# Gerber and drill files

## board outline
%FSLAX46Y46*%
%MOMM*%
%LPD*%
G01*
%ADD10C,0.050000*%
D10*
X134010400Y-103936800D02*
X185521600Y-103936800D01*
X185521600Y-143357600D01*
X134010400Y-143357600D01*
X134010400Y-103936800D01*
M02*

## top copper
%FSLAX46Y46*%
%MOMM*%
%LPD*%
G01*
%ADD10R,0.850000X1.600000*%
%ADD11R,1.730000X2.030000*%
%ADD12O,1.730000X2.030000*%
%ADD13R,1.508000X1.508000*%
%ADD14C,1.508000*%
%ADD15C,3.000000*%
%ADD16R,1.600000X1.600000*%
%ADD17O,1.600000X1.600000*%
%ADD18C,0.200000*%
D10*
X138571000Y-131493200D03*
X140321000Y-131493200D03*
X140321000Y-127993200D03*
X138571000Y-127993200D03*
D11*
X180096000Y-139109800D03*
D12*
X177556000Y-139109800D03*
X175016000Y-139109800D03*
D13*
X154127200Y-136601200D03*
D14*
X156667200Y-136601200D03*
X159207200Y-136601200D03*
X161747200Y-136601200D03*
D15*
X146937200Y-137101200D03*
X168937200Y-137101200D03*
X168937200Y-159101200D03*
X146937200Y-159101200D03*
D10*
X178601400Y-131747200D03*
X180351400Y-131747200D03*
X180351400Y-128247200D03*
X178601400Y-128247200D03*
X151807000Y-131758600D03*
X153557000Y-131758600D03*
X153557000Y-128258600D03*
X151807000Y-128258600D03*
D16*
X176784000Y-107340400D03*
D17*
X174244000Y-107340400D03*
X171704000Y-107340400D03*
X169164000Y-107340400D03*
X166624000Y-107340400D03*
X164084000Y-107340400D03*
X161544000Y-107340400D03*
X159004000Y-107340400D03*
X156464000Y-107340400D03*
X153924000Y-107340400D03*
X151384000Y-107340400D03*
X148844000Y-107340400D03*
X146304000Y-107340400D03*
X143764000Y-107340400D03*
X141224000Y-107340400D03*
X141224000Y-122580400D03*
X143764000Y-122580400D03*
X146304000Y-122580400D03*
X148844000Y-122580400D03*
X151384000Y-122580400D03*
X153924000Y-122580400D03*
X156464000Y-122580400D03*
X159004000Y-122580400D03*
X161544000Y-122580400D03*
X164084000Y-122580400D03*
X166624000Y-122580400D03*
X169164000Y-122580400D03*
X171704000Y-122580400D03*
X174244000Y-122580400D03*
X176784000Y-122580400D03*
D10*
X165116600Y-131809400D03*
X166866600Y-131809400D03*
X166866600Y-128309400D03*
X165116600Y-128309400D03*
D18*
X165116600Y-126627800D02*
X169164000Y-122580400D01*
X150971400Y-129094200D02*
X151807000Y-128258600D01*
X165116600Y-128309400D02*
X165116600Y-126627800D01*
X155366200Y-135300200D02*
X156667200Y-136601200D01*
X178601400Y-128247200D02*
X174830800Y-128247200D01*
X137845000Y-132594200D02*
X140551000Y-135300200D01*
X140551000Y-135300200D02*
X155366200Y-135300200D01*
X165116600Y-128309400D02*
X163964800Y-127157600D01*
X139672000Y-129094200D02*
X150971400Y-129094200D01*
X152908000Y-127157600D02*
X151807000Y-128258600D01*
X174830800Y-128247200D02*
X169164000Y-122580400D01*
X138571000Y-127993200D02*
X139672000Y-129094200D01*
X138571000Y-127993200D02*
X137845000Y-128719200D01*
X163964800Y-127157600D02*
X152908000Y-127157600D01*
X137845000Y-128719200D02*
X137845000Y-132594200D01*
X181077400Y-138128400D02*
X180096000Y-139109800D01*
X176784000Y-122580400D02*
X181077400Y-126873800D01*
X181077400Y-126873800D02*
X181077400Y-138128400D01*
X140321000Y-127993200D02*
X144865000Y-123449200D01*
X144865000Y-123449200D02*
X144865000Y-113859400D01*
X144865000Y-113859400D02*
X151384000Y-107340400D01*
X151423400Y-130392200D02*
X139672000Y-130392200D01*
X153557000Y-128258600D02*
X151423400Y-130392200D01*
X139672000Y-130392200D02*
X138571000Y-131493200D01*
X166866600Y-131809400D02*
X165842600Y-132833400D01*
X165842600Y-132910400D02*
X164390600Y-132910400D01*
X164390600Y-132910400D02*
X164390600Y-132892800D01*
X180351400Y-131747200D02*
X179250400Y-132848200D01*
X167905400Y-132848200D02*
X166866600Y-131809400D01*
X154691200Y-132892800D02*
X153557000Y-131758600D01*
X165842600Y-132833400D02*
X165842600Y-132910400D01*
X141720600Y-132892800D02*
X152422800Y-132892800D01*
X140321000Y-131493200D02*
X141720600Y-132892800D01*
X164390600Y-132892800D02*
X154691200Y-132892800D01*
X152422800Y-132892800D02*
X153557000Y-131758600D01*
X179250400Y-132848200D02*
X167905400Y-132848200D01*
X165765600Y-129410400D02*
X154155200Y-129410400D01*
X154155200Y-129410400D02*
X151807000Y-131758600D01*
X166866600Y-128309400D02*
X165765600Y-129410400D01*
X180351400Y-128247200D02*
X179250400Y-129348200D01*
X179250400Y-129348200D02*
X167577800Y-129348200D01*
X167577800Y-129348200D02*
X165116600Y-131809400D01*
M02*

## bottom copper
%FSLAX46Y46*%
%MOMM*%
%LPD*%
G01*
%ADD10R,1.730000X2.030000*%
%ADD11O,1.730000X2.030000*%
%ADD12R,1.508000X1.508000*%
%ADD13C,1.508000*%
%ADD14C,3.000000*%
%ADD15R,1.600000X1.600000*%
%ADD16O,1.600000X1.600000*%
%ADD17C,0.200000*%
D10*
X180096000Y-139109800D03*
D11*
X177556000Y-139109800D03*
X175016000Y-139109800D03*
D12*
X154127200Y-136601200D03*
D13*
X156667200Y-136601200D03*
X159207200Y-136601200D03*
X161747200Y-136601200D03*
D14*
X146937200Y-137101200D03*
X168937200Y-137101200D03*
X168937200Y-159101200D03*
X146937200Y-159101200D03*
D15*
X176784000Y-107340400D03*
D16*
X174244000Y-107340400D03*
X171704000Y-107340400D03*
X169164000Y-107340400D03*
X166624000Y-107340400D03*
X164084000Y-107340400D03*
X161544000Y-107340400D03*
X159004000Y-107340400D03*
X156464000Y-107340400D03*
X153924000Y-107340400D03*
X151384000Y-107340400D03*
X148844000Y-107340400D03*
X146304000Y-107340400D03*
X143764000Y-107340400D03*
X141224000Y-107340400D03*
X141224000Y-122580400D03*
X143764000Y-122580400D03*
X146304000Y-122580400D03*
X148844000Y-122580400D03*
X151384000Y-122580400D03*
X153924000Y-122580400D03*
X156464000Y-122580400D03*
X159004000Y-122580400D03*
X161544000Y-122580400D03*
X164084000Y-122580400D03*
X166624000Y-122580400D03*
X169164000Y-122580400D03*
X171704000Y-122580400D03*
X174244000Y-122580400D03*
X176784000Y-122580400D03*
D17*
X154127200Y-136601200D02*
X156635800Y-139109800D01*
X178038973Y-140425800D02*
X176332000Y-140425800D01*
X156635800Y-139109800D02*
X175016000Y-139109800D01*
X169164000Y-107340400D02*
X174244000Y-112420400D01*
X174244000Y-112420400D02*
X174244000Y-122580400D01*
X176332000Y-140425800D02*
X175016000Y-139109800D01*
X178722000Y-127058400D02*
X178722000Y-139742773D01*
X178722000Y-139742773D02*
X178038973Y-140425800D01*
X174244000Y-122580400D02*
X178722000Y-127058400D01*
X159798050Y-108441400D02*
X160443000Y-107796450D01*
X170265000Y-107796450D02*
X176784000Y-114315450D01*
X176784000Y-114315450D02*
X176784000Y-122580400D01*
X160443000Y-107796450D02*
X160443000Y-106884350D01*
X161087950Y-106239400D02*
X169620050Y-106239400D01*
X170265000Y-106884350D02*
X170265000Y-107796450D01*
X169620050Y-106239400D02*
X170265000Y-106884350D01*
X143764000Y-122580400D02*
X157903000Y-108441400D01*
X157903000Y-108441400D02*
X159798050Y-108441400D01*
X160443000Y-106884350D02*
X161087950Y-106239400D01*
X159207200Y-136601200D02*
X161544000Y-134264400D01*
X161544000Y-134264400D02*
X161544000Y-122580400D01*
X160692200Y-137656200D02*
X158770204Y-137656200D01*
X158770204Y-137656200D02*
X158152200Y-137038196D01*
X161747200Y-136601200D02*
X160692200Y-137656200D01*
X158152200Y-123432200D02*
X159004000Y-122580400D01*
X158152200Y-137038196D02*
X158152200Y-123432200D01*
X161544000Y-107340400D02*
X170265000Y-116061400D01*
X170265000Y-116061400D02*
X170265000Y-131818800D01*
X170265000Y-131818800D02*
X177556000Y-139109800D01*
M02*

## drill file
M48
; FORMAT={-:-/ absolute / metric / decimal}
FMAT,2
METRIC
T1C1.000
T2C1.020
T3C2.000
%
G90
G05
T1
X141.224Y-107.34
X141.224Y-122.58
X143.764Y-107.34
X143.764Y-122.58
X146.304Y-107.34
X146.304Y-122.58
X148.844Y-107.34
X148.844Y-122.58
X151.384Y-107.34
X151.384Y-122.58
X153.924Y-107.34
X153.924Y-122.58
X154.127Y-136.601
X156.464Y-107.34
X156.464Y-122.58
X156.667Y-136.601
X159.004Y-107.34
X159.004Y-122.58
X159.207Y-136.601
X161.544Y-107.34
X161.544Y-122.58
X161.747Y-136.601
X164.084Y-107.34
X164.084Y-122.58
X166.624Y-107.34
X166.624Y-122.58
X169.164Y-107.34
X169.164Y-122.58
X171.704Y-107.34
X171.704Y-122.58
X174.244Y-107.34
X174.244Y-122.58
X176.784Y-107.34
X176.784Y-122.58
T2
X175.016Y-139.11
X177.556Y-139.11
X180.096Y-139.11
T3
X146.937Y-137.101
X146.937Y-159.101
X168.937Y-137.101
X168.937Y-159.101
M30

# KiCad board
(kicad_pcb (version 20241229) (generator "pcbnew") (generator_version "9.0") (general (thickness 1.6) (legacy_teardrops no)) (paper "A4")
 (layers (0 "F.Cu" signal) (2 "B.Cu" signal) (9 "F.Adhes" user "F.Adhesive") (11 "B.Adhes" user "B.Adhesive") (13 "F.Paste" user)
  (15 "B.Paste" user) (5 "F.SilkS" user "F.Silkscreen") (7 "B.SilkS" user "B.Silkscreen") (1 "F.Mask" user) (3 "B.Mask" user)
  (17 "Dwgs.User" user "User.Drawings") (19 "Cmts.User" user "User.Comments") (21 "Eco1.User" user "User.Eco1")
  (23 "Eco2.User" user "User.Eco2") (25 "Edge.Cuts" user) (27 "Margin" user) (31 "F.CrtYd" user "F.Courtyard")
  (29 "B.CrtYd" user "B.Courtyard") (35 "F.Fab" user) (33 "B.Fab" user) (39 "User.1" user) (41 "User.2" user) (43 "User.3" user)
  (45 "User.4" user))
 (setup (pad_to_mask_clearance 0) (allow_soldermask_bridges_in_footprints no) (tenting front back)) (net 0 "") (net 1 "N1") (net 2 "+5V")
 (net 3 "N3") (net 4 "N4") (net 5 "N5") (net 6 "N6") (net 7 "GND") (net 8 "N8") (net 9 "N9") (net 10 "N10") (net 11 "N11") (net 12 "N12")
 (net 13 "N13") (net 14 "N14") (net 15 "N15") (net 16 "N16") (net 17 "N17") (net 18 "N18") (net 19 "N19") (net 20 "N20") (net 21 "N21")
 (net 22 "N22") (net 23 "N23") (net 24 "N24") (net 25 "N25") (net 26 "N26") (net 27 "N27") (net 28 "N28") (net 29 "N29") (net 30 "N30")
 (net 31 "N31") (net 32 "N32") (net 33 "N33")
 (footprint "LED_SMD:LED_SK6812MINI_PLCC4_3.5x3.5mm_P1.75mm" (layer "F.Cu") (at 139.446 129.7432 90)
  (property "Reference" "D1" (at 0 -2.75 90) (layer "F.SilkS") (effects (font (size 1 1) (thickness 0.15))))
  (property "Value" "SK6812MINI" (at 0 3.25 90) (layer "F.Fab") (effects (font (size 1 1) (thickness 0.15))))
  (pad "1" smd rect (at -1.75 -0.875 90) (size 1.6 0.85) (layers "F.Cu" "F.Mask" "F.Paste") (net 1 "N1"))
  (pad "2" smd rect (at -1.75 0.875 90) (size 1.6 0.85) (layers "F.Cu" "F.Mask" "F.Paste") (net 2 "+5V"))
  (pad "3" smd rect (at 1.75 0.875 90) (size 1.6 0.85) (layers "F.Cu" "F.Mask" "F.Paste") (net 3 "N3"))
  (pad "4" smd rect (at 1.75 -0.875 90) (size 1.6 0.85) (layers "F.Cu" "F.Mask" "F.Paste") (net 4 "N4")))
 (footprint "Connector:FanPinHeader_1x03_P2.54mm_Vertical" (layer "F.Cu") (at 180.096 139.1098 180)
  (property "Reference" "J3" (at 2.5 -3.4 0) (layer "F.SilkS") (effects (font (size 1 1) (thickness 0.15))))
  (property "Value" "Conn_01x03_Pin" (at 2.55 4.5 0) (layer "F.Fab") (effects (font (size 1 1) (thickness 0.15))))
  (pad "1" thru_hole rect (at 0 0 270) (size 2.03 1.73) (drill 1.02) (layers "*.Cu" "*.Mask") (remove_unused_layers no) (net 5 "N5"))
  (pad "2" thru_hole oval (at 2.54 0 270) (size 2.03 1.73) (drill 1.02) (layers "*.Cu" "*.Mask") (remove_unused_layers no) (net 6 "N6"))
  (pad "3" thru_hole oval (at 5.08 0 270) (size 2.03 1.73) (drill 1.02) (layers "*.Cu" "*.Mask") (remove_unused_layers no) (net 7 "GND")))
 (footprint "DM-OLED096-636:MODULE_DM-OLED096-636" (layer "F.Cu") (at 157.9372 148.1012)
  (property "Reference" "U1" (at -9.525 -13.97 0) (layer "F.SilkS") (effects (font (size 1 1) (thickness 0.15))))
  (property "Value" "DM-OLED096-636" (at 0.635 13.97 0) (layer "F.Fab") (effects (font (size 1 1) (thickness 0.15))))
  (pad "1" thru_hole rect (at -3.81 -11.5) (size 1.508 1.508) (drill 1) (layers "*.Cu" "*.Mask") (remove_unused_layers no) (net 7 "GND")
   (solder_mask_margin 0.102))
  (pad "2" thru_hole circle (at -1.27 -11.5) (size 1.508 1.508) (drill 1) (layers "*.Cu" "*.Mask") (remove_unused_layers no) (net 4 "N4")
   (solder_mask_margin 0.102))
  (pad "3" thru_hole circle (at 1.27 -11.5) (size 1.508 1.508) (drill 1) (layers "*.Cu" "*.Mask") (remove_unused_layers no) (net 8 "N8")
   (solder_mask_margin 0.102))
  (pad "4" thru_hole circle (at 3.81 -11.5) (size 1.508 1.508) (drill 1) (layers "*.Cu" "*.Mask") (remove_unused_layers no) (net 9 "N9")
   (solder_mask_margin 0.102))
  (pad "S1" thru_hole circle (at -11 -11) (size 3 3) (drill 2) (layers "*.Cu" "*.Mask") (remove_unused_layers no) (solder_mask_margin 0.102))
  (pad "S2" thru_hole circle (at 11 -11) (size 3 3) (drill 2) (layers "*.Cu" "*.Mask") (remove_unused_layers no) (solder_mask_margin 0.102))
  (pad "S3" thru_hole circle (at 11 11) (size 3 3) (drill 2) (layers "*.Cu" "*.Mask") (remove_unused_layers no) (solder_mask_margin 0.102))
  (pad "S4" thru_hole circle (at -11 11) (size 3 3) (drill 2) (layers "*.Cu" "*.Mask") (remove_unused_layers no) (solder_mask_margin 0.102)))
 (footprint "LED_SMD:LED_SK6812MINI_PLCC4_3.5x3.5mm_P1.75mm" (layer "F.Cu") (at 179.4764 129.9972 90)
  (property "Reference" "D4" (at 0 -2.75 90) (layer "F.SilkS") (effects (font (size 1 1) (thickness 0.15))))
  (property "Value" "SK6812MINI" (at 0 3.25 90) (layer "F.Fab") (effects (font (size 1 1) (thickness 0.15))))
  (pad "1" smd rect (at -1.75 -0.875 90) (size 1.6 0.85) (layers "F.Cu" "F.Mask" "F.Paste") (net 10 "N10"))
  (pad "2" smd rect (at -1.75 0.875 90) (size 1.6 0.85) (layers "F.Cu" "F.Mask" "F.Paste") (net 2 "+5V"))
  (pad "3" smd rect (at 1.75 0.875 90) (size 1.6 0.85) (layers "F.Cu" "F.Mask" "F.Paste") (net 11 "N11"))
  (pad "4" smd rect (at 1.75 -0.875 90) (size 1.6 0.85) (layers "F.Cu" "F.Mask" "F.Paste") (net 4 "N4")))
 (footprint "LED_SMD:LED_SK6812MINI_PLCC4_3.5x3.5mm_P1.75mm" (layer "F.Cu") (at 152.682 130.0086 90)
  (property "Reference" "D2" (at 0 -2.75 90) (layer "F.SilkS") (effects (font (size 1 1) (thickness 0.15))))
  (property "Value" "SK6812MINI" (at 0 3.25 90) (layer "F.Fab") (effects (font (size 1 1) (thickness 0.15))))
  (pad "1" smd rect (at -1.75 -0.875 90) (size 1.6 0.85) (layers "F.Cu" "F.Mask" "F.Paste") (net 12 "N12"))
  (pad "2" smd rect (at -1.75 0.875 90) (size 1.6 0.85) (layers "F.Cu" "F.Mask" "F.Paste") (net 2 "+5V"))
  (pad "3" smd rect (at 1.75 0.875 90) (size 1.6 0.85) (layers "F.Cu" "F.Mask" "F.Paste") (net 1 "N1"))
  (pad "4" smd rect (at 1.75 -0.875 90) (size 1.6 0.85) (layers "F.Cu" "F.Mask" "F.Paste") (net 4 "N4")))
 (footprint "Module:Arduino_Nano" (layer "F.Cu") (at 176.784 107.3404 -90)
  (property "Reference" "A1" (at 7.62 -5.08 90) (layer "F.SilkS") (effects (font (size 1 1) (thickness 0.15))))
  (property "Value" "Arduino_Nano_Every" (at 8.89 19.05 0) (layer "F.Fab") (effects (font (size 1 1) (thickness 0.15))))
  (pad "1" thru_hole rect (at 0 0 270) (size 1.6 1.6) (drill 1) (layers "*.Cu" "*.Mask") (remove_unused_layers no) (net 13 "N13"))
  (pad "2" thru_hole oval (at 0 2.54 270) (size 1.6 1.6) (drill 1) (layers "*.Cu" "*.Mask") (remove_unused_layers no) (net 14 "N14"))
  (pad "3" thru_hole oval (at 0 5.08 270) (size 1.6 1.6) (drill 1) (layers "*.Cu" "*.Mask") (remove_unused_layers no) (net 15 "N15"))
  (pad "4" thru_hole oval (at 0 7.62 270) (size 1.6 1.6) (drill 1) (layers "*.Cu" "*.Mask") (remove_unused_layers no) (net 7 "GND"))
  (pad "5" thru_hole oval (at 0 10.16 270) (size 1.6 1.6) (drill 1) (layers "*.Cu" "*.Mask") (remove_unused_layers no) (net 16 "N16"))
  (pad "6" thru_hole oval (at 0 12.7 270) (size 1.6 1.6) (drill 1) (layers "*.Cu" "*.Mask") (remove_unused_layers no) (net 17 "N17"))
  (pad "7" thru_hole oval (at 0 15.24 270) (size 1.6 1.6) (drill 1) (layers "*.Cu" "*.Mask") (remove_unused_layers no) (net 6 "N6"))
  (pad "8" thru_hole oval (at 0 17.78 270) (size 1.6 1.6) (drill 1) (layers "*.Cu" "*.Mask") (remove_unused_layers no) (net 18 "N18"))
  (pad "9" thru_hole oval (at 0 20.32 270) (size 1.6 1.6) (drill 1) (layers "*.Cu" "*.Mask") (remove_unused_layers no) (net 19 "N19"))
  (pad "10" thru_hole oval (at 0 22.86 270) (size 1.6 1.6) (drill 1) (layers "*.Cu" "*.Mask") (remove_unused_layers no) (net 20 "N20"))
  (pad "11" thru_hole oval (at 0 25.4 270) (size 1.6 1.6) (drill 1) (layers "*.Cu" "*.Mask") (remove_unused_layers no) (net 3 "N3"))
  (pad "12" thru_hole oval (at 0 27.94 270) (size 1.6 1.6) (drill 1) (layers "*.Cu" "*.Mask") (remove_unused_layers no) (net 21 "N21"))
  (pad "13" thru_hole oval (at 0 30.48 270) (size 1.6 1.6) (drill 1) (layers "*.Cu" "*.Mask") (remove_unused_layers no) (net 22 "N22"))
  (pad "14" thru_hole oval (at 0 33.02 270) (size 1.6 1.6) (drill 1) (layers "*.Cu" "*.Mask") (remove_unused_layers no) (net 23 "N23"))
  (pad "15" thru_hole oval (at 0 35.56 270) (size 1.6 1.6) (drill 1) (layers "*.Cu" "*.Mask") (remove_unused_layers no) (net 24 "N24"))
  (pad "16" thru_hole oval (at 15.24 35.56 270) (size 1.6 1.6) (drill 1) (layers "*.Cu" "*.Mask") (remove_unused_layers no) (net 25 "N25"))
  (pad "17" thru_hole oval (at 15.24 33.02 270) (size 1.6 1.6) (drill 1) (layers "*.Cu" "*.Mask") (remove_unused_layers no) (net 5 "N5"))
  (pad "18" thru_hole oval (at 15.24 30.48 270) (size 1.6 1.6) (drill 1) (layers "*.Cu" "*.Mask") (remove_unused_layers no) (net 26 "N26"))
  (pad "19" thru_hole oval (at 15.24 27.94 270) (size 1.6 1.6) (drill 1) (layers "*.Cu" "*.Mask") (remove_unused_layers no) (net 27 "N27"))
  (pad "20" thru_hole oval (at 15.24 25.4 270) (size 1.6 1.6) (drill 1) (layers "*.Cu" "*.Mask") (remove_unused_layers no) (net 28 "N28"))
  (pad "21" thru_hole oval (at 15.24 22.86 270) (size 1.6 1.6) (drill 1) (layers "*.Cu" "*.Mask") (remove_unused_layers no) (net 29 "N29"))
  (pad "22" thru_hole oval (at 15.24 20.32 270) (size 1.6 1.6) (drill 1) (layers "*.Cu" "*.Mask") (remove_unused_layers no) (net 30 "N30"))
  (pad "23" thru_hole oval (at 15.24 17.78 270) (size 1.6 1.6) (drill 1) (layers "*.Cu" "*.Mask") (remove_unused_layers no) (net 9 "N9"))
  (pad "24" thru_hole oval (at 15.24 15.24 270) (size 1.6 1.6) (drill 1) (layers "*.Cu" "*.Mask") (remove_unused_layers no) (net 8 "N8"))
  (pad "25" thru_hole oval (at 15.24 12.7 270) (size 1.6 1.6) (drill 1) (layers "*.Cu" "*.Mask") (remove_unused_layers no) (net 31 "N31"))
  (pad "26" thru_hole oval (at 15.24 10.16 270) (size 1.6 1.6) (drill 1) (layers "*.Cu" "*.Mask") (remove_unused_layers no) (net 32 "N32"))
  (pad "27" thru_hole oval (at 15.24 7.62 270) (size 1.6 1.6) (drill 1) (layers "*.Cu" "*.Mask") (remove_unused_layers no) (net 4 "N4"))
  (pad "28" thru_hole oval (at 15.24 5.08 270) (size 1.6 1.6) (drill 1) (layers "*.Cu" "*.Mask") (remove_unused_layers no) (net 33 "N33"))
  (pad "29" thru_hole oval (at 15.24 2.54 270) (size 1.6 1.6) (drill 1) (layers "*.Cu" "*.Mask") (remove_unused_layers no) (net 7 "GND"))
  (pad "30" thru_hole oval (at 15.24 0 270) (size 1.6 1.6) (drill 1) (layers "*.Cu" "*.Mask") (remove_unused_layers no) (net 5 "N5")))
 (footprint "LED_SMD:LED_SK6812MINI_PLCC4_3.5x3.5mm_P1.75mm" (layer "F.Cu") (at 165.9916 130.0594 90)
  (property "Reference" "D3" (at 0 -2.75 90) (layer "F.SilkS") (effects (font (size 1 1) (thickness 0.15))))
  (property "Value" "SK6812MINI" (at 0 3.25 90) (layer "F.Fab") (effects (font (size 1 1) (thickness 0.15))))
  (pad "1" smd rect (at -1.75 -0.875 90) (size 1.6 0.85) (layers "F.Cu" "F.Mask" "F.Paste") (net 11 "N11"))
  (pad "2" smd rect (at -1.75 0.875 90) (size 1.6 0.85) (layers "F.Cu" "F.Mask" "F.Paste") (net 2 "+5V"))
  (pad "3" smd rect (at 1.75 0.875 90) (size 1.6 0.85) (layers "F.Cu" "F.Mask" "F.Paste") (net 12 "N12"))
  (pad "4" smd rect (at 1.75 -0.875 90) (size 1.6 0.85) (layers "F.Cu" "F.Mask" "F.Paste") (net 4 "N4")))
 (gr_rect (start 134.0104 103.9368) (end 185.5216 143.3576) (stroke (width 0.05) (type default)) (fill no) (layer "Edge.Cuts"))
 (segment (start 154.1272 136.6012) (end 156.6358 139.1098) (width 0.2) (layer "B.Cu") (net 7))
 (segment (start 178.038973 140.4258) (end 176.332 140.4258) (width 0.2) (layer "B.Cu") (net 7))
 (segment (start 156.6358 139.1098) (end 175.016 139.1098) (width 0.2) (layer "B.Cu") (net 7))
 (segment (start 169.164 107.3404) (end 174.244 112.4204) (width 0.2) (layer "B.Cu") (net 7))
 (segment (start 174.244 112.4204) (end 174.244 122.5804) (width 0.2) (layer "B.Cu") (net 7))
 (segment (start 176.332 140.4258) (end 175.016 139.1098) (width 0.2) (layer "B.Cu") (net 7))
 (segment (start 178.722 127.0584) (end 178.722 139.742773) (width 0.2) (layer "B.Cu") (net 7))
 (segment (start 178.722 139.742773) (end 178.038973 140.4258) (width 0.2) (layer "B.Cu") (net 7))
 (segment (start 174.244 122.5804) (end 178.722 127.0584) (width 0.2) (layer "B.Cu") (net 7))
 (segment (start 165.1166 126.6278) (end 169.164 122.5804) (width 0.2) (layer "F.Cu") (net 4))
 (segment (start 150.9714 129.0942) (end 151.807 128.2586) (width 0.2) (layer "F.Cu") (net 4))
 (segment (start 165.1166 128.3094) (end 165.1166 126.6278) (width 0.2) (layer "F.Cu") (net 4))
 (segment (start 155.3662 135.3002) (end 156.6672 136.6012) (width 0.2) (layer "F.Cu") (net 4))
 (segment (start 178.6014 128.2472) (end 174.8308 128.2472) (width 0.2) (layer "F.Cu") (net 4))
 (segment (start 137.845 132.5942) (end 140.551 135.3002) (width 0.2) (layer "F.Cu") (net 4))
 (segment (start 140.551 135.3002) (end 155.3662 135.3002) (width 0.2) (layer "F.Cu") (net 4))
 (segment (start 165.1166 128.3094) (end 163.9648 127.1576) (width 0.2) (layer "F.Cu") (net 4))
 (segment (start 139.672 129.0942) (end 150.9714 129.0942) (width 0.2) (layer "F.Cu") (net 4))
 (segment (start 152.908 127.1576) (end 151.807 128.2586) (width 0.2) (layer "F.Cu") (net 4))
 (segment (start 174.8308 128.2472) (end 169.164 122.5804) (width 0.2) (layer "F.Cu") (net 4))
 (segment (start 138.571 127.9932) (end 139.672 129.0942) (width 0.2) (layer "F.Cu") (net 4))
 (segment (start 138.571 127.9932) (end 137.845 128.7192) (width 0.2) (layer "F.Cu") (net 4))
 (segment (start 163.9648 127.1576) (end 152.908 127.1576) (width 0.2) (layer "F.Cu") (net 4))
 (segment (start 137.845 128.7192) (end 137.845 132.5942) (width 0.2) (layer "F.Cu") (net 4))
 (segment (start 181.0774 138.1284) (end 180.096 139.1098) (width 0.2) (layer "F.Cu") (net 5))
 (segment (start 176.784 122.5804) (end 181.0774 126.8738) (width 0.2) (layer "F.Cu") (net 5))
 (segment (start 181.0774 126.8738) (end 181.0774 138.1284) (width 0.2) (layer "F.Cu") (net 5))
 (segment (start 159.79805 108.4414) (end 160.443 107.79645) (width 0.2) (layer "B.Cu") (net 5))
 (segment (start 170.265 107.79645) (end 176.784 114.31545) (width 0.2) (layer "B.Cu") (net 5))
 (segment (start 176.784 114.31545) (end 176.784 122.5804) (width 0.2) (layer "B.Cu") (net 5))
 (segment (start 160.443 107.79645) (end 160.443 106.88435) (width 0.2) (layer "B.Cu") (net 5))
 (segment (start 161.08795 106.2394) (end 169.62005 106.2394) (width 0.2) (layer "B.Cu") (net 5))
 (segment (start 170.265 106.88435) (end 170.265 107.79645) (width 0.2) (layer "B.Cu") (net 5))
 (segment (start 169.62005 106.2394) (end 170.265 106.88435) (width 0.2) (layer "B.Cu") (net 5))
 (segment (start 143.764 122.5804) (end 157.903 108.4414) (width 0.2) (layer "B.Cu") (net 5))
 (segment (start 157.903 108.4414) (end 159.79805 108.4414) (width 0.2) (layer "B.Cu") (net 5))
 (segment (start 160.443 106.88435) (end 161.08795 106.2394) (width 0.2) (layer "B.Cu") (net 5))
 (segment (start 159.2072 136.6012) (end 161.544 134.2644) (width 0.2) (layer "B.Cu") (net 8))
 (segment (start 161.544 134.2644) (end 161.544 122.5804) (width 0.2) (layer "B.Cu") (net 8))
 (segment (start 160.6922 137.6562) (end 158.770204 137.6562) (width 0.2) (layer "B.Cu") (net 9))
 (segment (start 158.770204 137.6562) (end 158.1522 137.038196) (width 0.2) (layer "B.Cu") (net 9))
 (segment (start 161.7472 136.6012) (end 160.6922 137.6562) (width 0.2) (layer "B.Cu") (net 9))
 (segment (start 158.1522 123.4322) (end 159.004 122.5804) (width 0.2) (layer "B.Cu") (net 9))
 (segment (start 158.1522 137.038196) (end 158.1522 123.4322) (width 0.2) (layer "B.Cu") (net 9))
 (segment (start 161.544 107.3404) (end 170.265 116.0614) (width 0.2) (layer "B.Cu") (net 6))
 (segment (start 170.265 116.0614) (end 170.265 131.8188) (width 0.2) (layer "B.Cu") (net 6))
 (segment (start 170.265 131.8188) (end 177.556 139.1098) (width 0.2) (layer "B.Cu") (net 6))
 (segment (start 140.321 127.9932) (end 144.865 123.4492) (width 0.2) (layer "F.Cu") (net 3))
 (segment (start 144.865 123.4492) (end 144.865 113.8594) (width 0.2) (layer "F.Cu") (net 3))
 (segment (start 144.865 113.8594) (end 151.384 107.3404) (width 0.2) (layer "F.Cu") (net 3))
 (segment (start 151.4234 130.3922) (end 139.672 130.3922) (width 0.2) (layer "F.Cu") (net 1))
 (segment (start 153.557 128.2586) (end 151.4234 130.3922) (width 0.2) (layer "F.Cu") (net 1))
 (segment (start 139.672 130.3922) (end 138.571 131.4932) (width 0.2) (layer "F.Cu") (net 1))
 (segment (start 166.8666 131.8094) (end 165.8426 132.8334) (width 0.2) (layer "F.Cu") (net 2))
 (segment (start 165.8426 132.9104) (end 164.3906 132.9104) (width 0.2) (layer "F.Cu") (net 2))
 (segment (start 164.3906 132.9104) (end 164.3906 132.8928) (width 0.2) (layer "F.Cu") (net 2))
 (segment (start 180.3514 131.7472) (end 179.2504 132.8482) (width 0.2) (layer "F.Cu") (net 2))
 (segment (start 167.9054 132.8482) (end 166.8666 131.8094) (width 0.2) (layer "F.Cu") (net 2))
 (segment (start 154.6912 132.8928) (end 153.557 131.7586) (width 0.2) (layer "F.Cu") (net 2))
 (segment (start 165.8426 132.8334) (end 165.8426 132.9104) (width 0.2) (layer "F.Cu") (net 2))
 (segment (start 141.7206 132.8928) (end 152.4228 132.8928) (width 0.2) (layer "F.Cu") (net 2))
 (segment (start 140.321 131.4932) (end 141.7206 132.8928) (width 0.2) (layer "F.Cu") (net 2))
 (segment (start 164.3906 132.8928) (end 154.6912 132.8928) (width 0.2) (layer "F.Cu") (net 2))
 (segment (start 152.4228 132.8928) (end 153.557 131.7586) (width 0.2) (layer "F.Cu") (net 2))
 (segment (start 179.2504 132.8482) (end 167.9054 132.8482) (width 0.2) (layer "F.Cu") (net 2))
 (segment (start 165.7656 129.4104) (end 154.1552 129.4104) (width 0.2) (layer "F.Cu") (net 12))
 (segment (start 154.1552 129.4104) (end 151.807 131.7586) (width 0.2) (layer "F.Cu") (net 12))
 (segment (start 166.8666 128.3094) (end 165.7656 129.4104) (width 0.2) (layer "F.Cu") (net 12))
 (segment (start 180.3514 128.2472) (end 179.2504 129.3482) (width 0.2) (layer "F.Cu") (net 11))
 (segment (start 179.2504 129.3482) (end 167.5778 129.3482) (width 0.2) (layer "F.Cu") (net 11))
 (segment (start 167.5778 129.3482) (end 165.1166 131.8094) (width 0.2) (layer "F.Cu") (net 11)))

